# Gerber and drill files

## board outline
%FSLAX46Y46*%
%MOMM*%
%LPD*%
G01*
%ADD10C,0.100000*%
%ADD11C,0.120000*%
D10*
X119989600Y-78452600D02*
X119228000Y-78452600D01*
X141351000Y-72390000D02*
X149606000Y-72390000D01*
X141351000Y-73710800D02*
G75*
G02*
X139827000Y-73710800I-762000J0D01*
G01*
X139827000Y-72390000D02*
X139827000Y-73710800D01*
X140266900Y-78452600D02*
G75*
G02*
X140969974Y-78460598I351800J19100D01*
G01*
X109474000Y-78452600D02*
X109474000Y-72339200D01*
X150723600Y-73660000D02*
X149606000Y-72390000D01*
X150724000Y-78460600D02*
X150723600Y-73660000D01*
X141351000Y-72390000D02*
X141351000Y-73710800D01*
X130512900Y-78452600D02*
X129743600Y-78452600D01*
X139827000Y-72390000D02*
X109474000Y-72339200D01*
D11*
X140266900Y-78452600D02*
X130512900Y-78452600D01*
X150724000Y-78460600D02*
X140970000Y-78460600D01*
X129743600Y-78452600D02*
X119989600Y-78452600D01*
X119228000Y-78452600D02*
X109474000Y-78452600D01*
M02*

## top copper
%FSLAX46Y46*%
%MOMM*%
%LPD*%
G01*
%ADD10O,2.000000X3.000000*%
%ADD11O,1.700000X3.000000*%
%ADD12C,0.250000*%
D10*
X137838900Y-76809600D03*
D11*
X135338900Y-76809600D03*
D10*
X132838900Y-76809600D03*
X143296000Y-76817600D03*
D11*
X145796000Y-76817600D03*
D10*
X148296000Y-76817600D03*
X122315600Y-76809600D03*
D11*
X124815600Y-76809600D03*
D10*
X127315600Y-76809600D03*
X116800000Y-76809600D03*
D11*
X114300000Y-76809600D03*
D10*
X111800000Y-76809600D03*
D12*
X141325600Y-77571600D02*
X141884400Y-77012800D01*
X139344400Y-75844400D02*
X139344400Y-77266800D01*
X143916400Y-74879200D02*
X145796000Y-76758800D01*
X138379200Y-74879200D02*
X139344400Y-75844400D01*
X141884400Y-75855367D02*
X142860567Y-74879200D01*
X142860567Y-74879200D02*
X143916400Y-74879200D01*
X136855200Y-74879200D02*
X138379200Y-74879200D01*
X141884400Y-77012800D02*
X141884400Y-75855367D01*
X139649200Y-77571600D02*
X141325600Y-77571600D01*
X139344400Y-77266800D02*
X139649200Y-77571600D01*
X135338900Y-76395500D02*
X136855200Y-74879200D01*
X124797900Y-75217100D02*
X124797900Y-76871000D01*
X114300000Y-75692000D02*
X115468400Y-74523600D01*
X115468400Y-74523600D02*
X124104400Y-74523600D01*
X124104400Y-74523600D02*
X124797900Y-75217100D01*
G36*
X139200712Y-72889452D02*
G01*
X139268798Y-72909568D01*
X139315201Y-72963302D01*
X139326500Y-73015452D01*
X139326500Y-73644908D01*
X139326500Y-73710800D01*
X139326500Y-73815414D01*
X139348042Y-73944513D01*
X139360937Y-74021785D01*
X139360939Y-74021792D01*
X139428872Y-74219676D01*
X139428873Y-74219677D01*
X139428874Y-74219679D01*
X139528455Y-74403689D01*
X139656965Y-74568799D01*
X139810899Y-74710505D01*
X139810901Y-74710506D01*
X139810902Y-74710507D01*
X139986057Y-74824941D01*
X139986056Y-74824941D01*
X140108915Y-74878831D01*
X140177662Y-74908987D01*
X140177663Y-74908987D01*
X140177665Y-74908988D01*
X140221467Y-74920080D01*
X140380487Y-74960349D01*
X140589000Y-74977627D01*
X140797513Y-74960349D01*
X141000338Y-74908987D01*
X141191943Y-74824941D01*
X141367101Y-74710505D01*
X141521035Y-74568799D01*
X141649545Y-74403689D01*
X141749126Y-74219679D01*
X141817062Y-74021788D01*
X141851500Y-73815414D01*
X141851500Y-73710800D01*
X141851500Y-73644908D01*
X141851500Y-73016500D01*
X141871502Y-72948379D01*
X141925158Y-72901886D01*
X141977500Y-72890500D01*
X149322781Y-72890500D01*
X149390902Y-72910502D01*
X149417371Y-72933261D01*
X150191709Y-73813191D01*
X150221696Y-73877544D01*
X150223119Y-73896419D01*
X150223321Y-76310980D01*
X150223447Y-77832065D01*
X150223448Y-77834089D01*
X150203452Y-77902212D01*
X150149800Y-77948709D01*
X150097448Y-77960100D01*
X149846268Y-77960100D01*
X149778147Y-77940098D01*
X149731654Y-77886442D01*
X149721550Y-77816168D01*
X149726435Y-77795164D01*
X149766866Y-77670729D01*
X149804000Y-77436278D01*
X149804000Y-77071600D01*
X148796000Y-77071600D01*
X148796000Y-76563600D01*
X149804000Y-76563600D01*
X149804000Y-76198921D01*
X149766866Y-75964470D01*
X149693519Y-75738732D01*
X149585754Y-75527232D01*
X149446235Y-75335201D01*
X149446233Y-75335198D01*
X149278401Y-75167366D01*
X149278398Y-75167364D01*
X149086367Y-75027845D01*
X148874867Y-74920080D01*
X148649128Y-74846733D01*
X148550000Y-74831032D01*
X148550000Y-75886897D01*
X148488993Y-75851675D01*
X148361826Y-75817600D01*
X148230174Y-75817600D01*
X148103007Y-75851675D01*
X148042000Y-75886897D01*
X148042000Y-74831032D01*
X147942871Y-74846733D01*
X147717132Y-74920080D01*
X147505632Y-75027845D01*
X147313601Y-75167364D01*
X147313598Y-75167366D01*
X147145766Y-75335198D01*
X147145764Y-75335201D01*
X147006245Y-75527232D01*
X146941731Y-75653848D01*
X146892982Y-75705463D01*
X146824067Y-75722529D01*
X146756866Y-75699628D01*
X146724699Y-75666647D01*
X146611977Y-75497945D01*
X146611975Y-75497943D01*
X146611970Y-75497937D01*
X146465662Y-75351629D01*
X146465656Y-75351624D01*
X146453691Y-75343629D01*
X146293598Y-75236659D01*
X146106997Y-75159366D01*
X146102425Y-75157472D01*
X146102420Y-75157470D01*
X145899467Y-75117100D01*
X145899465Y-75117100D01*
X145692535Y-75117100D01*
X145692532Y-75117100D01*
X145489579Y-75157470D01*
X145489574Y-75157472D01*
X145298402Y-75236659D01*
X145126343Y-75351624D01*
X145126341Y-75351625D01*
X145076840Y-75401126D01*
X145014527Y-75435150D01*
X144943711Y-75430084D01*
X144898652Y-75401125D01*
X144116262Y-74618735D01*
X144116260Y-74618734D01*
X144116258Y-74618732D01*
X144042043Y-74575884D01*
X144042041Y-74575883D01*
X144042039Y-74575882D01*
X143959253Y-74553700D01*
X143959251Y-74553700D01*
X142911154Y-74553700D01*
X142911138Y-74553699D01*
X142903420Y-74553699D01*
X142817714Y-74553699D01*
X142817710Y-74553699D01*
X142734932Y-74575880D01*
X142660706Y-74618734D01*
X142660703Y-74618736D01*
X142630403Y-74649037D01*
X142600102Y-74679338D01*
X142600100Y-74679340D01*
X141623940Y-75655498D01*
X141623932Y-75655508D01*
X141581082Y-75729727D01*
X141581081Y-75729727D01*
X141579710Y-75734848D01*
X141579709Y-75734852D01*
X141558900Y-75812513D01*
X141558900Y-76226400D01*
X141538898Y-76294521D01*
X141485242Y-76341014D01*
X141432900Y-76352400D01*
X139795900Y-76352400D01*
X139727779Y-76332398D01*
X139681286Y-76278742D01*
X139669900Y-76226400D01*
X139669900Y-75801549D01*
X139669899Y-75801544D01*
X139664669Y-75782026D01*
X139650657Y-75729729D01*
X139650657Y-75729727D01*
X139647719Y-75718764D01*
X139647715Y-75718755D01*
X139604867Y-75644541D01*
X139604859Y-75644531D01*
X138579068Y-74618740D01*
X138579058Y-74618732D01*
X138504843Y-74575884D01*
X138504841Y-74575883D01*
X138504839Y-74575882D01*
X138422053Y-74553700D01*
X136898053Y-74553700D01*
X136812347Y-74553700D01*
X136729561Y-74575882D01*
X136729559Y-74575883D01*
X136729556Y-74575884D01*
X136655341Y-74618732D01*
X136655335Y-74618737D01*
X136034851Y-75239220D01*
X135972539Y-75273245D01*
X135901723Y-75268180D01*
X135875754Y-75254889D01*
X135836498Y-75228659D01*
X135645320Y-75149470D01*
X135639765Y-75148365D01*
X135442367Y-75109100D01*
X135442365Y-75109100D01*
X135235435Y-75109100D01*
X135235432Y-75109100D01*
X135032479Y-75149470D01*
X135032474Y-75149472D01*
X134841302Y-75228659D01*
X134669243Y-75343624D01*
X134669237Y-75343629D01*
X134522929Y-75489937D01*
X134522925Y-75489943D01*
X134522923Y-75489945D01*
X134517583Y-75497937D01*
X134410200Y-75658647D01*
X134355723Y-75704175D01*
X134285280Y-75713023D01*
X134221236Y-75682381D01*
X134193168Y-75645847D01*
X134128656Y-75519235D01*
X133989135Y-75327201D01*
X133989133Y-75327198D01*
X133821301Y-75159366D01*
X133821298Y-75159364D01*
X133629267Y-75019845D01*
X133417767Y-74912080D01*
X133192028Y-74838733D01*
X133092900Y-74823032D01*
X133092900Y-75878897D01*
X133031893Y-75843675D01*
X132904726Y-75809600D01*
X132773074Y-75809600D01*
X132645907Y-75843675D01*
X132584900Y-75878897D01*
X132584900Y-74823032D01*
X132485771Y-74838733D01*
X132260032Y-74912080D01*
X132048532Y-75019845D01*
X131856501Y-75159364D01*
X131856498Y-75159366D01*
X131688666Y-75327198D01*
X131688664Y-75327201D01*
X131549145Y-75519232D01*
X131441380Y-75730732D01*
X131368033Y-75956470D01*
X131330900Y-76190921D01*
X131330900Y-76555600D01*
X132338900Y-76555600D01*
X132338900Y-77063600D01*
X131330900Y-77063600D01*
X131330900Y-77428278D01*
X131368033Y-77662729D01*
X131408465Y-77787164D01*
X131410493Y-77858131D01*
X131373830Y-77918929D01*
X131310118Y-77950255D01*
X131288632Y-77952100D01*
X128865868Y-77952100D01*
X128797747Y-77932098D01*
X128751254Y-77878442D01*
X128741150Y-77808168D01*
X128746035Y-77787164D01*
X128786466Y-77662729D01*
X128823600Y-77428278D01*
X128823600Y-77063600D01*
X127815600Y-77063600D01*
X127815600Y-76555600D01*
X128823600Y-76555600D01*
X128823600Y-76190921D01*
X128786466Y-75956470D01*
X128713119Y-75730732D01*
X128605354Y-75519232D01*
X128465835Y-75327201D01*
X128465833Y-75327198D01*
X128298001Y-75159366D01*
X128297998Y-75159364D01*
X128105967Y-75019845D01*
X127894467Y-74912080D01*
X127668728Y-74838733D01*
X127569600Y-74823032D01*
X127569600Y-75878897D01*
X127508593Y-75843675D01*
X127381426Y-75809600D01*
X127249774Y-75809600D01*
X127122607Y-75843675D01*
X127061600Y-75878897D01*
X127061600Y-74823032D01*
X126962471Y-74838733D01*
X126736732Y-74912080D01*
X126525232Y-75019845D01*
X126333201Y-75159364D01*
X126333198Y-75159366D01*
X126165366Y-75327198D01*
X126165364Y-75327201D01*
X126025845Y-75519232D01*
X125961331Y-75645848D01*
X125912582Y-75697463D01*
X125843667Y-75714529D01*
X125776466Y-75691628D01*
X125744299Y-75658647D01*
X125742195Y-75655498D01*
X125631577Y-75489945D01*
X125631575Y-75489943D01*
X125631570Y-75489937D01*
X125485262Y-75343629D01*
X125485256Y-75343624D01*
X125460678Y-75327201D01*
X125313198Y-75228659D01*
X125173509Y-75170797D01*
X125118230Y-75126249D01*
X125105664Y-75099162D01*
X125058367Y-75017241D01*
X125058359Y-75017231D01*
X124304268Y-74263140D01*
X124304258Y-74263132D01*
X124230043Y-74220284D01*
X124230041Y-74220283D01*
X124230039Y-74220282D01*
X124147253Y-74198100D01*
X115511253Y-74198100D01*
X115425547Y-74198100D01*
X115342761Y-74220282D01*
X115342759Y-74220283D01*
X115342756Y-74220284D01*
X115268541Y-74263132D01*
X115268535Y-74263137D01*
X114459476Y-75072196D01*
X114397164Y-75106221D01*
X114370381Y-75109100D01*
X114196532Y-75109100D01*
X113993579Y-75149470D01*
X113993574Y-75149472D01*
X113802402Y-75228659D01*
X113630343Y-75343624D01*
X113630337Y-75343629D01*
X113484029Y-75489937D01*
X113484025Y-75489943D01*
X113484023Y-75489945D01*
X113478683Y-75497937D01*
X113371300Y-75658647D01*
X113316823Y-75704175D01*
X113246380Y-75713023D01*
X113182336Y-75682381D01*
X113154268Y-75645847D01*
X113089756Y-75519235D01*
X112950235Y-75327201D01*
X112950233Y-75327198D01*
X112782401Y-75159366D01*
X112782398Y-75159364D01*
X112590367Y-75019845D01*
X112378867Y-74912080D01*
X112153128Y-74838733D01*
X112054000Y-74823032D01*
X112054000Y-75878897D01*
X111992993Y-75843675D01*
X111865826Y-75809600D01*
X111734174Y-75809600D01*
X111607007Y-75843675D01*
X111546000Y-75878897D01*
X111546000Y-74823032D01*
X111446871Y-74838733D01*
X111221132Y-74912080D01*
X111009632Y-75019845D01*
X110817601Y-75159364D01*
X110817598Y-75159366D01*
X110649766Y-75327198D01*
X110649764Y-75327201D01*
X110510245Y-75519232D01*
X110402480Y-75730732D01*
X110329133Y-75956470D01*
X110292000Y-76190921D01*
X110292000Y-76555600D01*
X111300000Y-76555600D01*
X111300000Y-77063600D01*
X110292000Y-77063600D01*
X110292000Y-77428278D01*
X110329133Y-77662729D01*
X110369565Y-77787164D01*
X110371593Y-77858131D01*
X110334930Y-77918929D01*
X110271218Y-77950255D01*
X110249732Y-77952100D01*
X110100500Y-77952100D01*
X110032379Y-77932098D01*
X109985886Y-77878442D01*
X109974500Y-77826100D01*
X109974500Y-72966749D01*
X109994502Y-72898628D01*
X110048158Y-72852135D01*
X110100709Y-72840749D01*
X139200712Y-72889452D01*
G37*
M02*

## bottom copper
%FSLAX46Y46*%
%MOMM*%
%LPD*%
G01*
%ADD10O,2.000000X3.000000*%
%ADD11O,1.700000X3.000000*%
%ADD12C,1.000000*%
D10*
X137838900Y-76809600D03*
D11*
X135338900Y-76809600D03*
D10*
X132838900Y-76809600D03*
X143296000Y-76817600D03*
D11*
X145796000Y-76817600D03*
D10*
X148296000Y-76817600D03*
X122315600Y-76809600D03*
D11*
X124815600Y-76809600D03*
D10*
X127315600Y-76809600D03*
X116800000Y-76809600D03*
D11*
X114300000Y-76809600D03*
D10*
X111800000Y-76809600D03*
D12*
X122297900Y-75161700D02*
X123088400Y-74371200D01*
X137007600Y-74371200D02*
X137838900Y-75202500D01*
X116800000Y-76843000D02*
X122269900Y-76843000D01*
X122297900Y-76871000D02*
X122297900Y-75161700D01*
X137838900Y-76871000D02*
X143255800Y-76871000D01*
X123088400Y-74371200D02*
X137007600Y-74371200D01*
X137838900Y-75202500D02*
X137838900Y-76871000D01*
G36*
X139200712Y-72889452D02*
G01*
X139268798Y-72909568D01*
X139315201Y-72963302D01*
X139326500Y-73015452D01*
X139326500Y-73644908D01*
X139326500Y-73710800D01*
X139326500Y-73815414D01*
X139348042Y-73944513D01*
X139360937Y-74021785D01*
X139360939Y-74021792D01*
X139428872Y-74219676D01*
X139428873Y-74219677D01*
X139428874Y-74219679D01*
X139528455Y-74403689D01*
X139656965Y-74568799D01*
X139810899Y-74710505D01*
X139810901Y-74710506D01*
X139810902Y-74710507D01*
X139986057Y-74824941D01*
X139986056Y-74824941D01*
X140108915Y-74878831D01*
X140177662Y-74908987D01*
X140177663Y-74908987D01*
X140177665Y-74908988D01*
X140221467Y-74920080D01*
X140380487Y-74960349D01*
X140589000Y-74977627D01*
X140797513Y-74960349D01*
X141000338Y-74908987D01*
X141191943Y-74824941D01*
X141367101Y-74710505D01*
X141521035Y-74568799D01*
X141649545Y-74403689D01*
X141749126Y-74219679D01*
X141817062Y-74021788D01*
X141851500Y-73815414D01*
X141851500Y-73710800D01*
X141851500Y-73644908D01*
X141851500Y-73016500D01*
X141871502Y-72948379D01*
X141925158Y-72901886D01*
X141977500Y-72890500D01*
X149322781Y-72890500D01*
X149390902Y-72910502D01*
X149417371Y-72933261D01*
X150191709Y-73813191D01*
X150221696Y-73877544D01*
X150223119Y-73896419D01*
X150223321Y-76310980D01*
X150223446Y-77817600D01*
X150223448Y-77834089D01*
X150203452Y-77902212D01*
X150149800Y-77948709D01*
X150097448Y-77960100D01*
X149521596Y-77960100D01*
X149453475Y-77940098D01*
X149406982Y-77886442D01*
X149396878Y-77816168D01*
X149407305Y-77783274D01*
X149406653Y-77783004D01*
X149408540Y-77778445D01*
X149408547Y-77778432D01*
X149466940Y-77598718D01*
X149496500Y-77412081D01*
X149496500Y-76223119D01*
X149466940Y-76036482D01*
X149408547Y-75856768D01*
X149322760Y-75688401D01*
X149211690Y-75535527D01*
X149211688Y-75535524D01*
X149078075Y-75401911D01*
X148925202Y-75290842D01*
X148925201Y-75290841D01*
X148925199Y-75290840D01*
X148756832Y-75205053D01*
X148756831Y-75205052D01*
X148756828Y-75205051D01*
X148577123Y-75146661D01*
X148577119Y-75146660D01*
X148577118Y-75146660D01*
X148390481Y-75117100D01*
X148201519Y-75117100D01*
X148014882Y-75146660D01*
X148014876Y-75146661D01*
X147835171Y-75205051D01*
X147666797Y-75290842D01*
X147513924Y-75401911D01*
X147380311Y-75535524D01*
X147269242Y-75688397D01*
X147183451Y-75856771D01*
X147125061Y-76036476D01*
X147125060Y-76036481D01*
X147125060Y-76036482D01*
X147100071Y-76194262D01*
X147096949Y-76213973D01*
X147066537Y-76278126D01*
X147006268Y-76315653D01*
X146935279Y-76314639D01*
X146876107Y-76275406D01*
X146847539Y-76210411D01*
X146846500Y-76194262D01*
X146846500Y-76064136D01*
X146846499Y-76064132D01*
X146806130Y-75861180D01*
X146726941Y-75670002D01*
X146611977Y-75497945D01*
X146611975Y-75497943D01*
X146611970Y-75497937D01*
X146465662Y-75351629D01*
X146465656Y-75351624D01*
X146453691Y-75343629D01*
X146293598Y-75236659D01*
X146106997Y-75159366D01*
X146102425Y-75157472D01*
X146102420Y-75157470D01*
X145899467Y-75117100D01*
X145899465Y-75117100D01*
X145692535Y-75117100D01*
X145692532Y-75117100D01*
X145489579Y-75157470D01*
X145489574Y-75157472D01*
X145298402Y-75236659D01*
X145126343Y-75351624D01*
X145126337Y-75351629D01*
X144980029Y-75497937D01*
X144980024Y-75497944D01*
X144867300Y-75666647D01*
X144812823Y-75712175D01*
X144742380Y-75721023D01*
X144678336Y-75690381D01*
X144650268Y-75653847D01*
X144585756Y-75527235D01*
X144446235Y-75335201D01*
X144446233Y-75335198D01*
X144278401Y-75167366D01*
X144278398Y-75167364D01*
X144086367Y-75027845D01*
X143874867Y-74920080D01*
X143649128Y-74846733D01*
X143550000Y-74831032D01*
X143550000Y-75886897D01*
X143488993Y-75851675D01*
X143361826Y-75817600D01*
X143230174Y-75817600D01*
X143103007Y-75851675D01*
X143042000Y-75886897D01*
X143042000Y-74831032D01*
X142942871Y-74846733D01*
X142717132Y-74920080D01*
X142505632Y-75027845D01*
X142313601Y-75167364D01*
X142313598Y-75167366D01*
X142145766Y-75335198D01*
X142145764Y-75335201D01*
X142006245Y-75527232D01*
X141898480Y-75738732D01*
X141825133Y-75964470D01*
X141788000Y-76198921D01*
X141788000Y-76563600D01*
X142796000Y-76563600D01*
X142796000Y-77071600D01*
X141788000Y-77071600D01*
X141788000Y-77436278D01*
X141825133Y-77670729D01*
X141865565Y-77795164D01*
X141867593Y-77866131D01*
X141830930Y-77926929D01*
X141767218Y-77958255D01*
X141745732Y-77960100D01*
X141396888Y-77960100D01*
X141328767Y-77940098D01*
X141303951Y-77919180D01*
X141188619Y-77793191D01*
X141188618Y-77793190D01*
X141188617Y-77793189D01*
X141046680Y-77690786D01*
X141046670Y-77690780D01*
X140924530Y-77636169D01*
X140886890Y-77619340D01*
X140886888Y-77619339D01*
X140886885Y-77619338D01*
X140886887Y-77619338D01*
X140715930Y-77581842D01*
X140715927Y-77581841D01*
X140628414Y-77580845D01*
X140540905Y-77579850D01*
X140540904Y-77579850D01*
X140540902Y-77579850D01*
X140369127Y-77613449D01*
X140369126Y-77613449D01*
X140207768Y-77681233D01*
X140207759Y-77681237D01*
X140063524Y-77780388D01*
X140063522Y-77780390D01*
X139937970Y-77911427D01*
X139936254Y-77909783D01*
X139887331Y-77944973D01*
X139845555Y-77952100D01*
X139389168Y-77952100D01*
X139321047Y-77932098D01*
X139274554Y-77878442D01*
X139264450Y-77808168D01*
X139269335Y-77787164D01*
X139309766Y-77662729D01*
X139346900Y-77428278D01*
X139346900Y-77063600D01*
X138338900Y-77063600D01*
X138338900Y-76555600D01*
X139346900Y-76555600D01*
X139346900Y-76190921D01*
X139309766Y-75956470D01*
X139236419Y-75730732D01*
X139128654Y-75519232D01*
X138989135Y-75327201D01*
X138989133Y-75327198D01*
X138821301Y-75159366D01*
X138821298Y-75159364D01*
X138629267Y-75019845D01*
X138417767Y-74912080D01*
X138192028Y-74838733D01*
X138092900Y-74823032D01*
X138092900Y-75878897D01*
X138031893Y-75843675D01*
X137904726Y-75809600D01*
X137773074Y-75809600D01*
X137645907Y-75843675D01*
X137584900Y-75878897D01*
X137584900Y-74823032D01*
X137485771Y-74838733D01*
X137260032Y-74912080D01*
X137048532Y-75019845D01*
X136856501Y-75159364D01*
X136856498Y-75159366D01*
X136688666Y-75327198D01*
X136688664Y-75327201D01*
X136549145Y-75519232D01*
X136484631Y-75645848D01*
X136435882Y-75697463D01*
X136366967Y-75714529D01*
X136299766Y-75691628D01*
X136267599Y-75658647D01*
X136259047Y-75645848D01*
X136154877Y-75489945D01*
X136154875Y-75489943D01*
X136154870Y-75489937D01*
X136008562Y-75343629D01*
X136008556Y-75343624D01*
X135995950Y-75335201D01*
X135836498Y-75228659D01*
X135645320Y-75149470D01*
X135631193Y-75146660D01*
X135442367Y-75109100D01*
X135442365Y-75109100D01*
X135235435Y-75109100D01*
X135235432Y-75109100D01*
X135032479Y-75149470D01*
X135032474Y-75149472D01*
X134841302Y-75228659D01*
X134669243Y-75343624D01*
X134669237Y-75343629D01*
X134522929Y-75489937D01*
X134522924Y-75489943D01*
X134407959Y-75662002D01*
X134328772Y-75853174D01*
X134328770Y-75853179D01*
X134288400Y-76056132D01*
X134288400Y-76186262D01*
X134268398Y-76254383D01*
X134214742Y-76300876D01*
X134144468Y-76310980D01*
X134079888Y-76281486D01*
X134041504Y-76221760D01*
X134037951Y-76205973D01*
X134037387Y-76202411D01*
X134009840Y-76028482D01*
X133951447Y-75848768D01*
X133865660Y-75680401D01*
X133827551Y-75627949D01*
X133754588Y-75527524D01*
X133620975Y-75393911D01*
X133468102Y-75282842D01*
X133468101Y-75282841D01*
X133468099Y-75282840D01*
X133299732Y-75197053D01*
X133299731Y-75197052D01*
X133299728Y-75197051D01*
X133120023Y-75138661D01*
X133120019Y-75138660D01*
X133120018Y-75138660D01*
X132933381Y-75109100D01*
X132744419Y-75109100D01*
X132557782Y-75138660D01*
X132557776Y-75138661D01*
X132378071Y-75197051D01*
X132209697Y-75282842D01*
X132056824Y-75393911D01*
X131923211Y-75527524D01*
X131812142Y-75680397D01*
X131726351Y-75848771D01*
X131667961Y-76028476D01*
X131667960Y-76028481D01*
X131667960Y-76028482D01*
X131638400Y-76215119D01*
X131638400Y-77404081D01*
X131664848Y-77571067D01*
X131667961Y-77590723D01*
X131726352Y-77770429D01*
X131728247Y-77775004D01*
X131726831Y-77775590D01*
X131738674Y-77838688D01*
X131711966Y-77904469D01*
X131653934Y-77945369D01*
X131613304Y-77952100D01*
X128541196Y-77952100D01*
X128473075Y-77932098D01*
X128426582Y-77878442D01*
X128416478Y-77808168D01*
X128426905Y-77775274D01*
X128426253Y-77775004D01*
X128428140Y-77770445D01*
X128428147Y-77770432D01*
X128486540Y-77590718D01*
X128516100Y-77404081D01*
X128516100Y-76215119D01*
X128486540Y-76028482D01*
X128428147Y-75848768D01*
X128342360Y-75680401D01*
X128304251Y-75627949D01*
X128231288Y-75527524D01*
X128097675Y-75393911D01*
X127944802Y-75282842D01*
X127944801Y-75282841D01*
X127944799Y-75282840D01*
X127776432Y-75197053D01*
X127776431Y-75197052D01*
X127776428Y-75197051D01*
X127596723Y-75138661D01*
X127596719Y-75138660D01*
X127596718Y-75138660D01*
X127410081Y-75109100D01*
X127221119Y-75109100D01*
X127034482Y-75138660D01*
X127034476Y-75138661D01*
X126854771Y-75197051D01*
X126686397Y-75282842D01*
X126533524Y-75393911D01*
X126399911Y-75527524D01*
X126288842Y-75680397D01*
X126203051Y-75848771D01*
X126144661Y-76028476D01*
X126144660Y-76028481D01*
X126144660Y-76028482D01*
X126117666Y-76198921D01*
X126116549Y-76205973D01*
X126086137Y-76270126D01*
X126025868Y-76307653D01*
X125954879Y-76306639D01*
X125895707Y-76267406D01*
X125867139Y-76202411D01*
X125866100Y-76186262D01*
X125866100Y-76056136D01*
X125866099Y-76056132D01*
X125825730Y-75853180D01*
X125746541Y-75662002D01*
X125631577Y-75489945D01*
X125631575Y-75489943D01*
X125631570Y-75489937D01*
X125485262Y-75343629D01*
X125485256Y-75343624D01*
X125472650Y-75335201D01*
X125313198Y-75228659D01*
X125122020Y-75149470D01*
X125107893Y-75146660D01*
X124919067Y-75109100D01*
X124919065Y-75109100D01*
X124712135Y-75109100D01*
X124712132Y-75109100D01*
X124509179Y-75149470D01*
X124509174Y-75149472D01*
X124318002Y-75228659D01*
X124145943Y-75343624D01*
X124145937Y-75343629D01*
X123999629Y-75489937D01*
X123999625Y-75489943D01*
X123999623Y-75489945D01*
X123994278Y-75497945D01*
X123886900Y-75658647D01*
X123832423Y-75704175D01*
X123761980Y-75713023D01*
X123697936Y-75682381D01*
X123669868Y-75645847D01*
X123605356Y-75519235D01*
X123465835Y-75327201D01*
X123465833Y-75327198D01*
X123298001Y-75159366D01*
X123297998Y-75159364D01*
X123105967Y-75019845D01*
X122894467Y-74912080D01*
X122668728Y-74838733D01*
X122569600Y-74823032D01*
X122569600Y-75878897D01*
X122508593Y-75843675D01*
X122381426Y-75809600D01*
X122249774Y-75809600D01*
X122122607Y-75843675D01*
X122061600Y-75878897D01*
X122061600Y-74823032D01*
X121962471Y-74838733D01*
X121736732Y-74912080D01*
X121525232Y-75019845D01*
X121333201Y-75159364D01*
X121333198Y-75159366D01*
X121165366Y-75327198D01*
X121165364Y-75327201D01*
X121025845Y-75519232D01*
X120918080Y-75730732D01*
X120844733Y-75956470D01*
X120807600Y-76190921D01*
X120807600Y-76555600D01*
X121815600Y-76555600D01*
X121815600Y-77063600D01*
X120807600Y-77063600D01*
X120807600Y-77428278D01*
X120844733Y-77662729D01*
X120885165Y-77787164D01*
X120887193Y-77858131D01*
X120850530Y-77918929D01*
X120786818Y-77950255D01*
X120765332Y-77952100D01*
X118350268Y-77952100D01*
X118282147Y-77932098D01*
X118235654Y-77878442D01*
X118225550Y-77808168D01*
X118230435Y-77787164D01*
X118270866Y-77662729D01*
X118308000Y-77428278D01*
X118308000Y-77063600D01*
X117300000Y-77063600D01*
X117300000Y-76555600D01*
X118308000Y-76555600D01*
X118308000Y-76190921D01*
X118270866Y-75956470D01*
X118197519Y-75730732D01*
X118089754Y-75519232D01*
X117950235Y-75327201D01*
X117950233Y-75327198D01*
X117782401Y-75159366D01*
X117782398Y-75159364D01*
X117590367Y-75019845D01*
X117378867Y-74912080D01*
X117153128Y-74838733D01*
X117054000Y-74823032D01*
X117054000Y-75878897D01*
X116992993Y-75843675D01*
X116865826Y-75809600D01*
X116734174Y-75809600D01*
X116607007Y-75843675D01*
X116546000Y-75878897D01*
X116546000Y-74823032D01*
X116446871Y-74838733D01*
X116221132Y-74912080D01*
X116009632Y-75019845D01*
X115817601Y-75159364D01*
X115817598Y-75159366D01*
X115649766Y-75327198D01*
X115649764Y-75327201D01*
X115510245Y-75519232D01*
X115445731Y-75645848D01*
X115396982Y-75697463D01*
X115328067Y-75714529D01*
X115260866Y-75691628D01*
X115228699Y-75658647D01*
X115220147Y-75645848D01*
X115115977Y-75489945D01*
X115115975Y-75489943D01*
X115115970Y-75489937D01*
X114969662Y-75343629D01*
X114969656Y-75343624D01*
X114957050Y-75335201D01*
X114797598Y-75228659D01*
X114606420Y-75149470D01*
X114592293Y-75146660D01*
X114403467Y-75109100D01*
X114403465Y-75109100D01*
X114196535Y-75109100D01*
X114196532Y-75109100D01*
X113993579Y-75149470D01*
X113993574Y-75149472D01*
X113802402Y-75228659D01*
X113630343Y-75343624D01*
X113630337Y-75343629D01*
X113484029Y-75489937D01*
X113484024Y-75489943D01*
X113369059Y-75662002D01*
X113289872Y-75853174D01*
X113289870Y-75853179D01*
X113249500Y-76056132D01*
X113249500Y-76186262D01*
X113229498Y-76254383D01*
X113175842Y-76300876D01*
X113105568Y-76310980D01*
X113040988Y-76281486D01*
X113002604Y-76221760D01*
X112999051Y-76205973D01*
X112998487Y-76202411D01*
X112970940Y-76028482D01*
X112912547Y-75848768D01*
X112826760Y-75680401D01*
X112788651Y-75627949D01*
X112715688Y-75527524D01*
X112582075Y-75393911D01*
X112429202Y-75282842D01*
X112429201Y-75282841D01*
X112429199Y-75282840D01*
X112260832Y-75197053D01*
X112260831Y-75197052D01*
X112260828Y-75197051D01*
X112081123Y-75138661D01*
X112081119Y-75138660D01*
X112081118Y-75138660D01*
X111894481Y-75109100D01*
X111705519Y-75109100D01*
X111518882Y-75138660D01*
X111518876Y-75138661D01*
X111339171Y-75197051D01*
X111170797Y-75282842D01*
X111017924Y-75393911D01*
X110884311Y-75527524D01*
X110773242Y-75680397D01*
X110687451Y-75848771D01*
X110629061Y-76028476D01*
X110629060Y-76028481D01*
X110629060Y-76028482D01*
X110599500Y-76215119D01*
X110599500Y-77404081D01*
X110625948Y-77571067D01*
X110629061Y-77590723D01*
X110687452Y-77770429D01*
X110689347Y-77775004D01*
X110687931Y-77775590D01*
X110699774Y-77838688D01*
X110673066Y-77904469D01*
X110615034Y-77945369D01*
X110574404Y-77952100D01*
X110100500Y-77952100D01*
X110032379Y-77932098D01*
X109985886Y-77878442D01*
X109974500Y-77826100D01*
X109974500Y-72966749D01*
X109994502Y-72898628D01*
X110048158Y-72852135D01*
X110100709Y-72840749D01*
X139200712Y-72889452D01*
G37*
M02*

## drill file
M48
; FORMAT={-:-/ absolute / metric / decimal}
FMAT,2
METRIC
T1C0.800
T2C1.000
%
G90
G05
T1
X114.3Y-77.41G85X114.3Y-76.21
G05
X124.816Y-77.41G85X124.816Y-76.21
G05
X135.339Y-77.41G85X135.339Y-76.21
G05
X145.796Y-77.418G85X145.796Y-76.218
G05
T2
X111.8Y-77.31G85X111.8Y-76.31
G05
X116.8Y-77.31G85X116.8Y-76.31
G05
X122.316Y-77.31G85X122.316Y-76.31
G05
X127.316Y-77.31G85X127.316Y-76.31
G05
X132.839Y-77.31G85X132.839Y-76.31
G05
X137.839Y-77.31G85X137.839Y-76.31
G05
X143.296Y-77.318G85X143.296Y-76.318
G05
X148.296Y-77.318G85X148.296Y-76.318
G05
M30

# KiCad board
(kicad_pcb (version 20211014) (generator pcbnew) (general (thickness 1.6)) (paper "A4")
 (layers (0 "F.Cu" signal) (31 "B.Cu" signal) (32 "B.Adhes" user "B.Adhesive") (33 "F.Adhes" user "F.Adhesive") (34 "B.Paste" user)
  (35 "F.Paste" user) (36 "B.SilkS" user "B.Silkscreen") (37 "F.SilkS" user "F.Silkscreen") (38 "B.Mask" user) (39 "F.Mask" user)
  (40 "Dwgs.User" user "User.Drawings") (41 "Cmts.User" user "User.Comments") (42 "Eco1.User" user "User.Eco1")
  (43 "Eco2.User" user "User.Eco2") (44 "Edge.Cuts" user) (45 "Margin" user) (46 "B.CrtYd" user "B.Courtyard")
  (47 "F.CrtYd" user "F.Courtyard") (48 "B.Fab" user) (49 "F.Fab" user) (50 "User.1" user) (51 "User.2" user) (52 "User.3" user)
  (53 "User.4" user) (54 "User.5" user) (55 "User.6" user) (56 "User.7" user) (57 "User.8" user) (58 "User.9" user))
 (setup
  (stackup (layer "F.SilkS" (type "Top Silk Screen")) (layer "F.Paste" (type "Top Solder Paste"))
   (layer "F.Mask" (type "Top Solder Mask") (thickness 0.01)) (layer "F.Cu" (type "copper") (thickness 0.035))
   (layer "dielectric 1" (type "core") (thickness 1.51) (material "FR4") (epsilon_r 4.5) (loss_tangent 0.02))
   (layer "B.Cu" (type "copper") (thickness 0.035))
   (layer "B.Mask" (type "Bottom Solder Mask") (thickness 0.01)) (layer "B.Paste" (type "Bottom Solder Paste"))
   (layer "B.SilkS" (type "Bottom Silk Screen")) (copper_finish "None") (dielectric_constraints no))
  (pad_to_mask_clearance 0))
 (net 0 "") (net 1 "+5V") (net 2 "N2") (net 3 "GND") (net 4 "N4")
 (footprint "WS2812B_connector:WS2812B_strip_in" (layer "F.Cu") (at 135.3389 77.3096 180)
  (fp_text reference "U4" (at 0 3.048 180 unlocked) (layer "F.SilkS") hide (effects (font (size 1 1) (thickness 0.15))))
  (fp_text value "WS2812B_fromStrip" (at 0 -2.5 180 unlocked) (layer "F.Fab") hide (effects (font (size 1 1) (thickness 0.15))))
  (fp_line (start -4.928 -1.143) (end 4.826 -1.143) (layer "Edge.Cuts") (width 0.12))
  (pad "1" thru_hole oval (at -2.5 0.5 180) (size 2 3) (drill oval 1 2) (layers *.Cu *.Mask) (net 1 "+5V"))
  (pad "2" thru_hole oval (at 0 0.5 180) (size 1.7 3) (drill oval 0.8 2) (layers *.Cu *.Mask) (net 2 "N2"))
  (pad "3" thru_hole oval (at 2.5 0.5 180) (size 2 3) (drill oval 1 2) (layers *.Cu *.Mask) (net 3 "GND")))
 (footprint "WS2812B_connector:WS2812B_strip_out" (layer "F.Cu") (at 145.796 77.3176 180)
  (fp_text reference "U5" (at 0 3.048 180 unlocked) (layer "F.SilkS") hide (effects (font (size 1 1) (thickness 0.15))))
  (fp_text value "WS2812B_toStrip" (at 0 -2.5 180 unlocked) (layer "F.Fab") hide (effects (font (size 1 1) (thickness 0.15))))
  (fp_line (start -4.928 -1.143) (end 4.826 -1.143) (layer "Edge.Cuts") (width 0.12))
  (pad "1" thru_hole oval (at 2.5 0.5 180) (size 2 3) (drill oval 1 2) (layers *.Cu *.Mask) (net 1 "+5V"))
  (pad "2" thru_hole oval (at 0 0.5 180) (size 1.7 3) (drill oval 0.8 2) (layers *.Cu *.Mask) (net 2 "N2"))
  (pad "3" thru_hole oval (at -2.5 0.5 180) (size 2 3) (drill oval 1 2) (layers *.Cu *.Mask) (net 3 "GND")))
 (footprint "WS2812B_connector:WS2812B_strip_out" (layer "F.Cu") (at 124.8156 77.3096 180)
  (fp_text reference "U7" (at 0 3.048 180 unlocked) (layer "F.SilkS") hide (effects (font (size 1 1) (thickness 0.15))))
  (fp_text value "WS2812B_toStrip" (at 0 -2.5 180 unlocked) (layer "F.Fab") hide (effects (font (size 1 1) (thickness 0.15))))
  (fp_line (start -4.928 -1.143) (end 4.826 -1.143) (layer "Edge.Cuts") (width 0.12))
  (pad "1" thru_hole oval (at 2.5 0.5 180) (size 2 3) (drill oval 1 2) (layers *.Cu *.Mask) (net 1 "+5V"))
  (pad "2" thru_hole oval (at 0 0.5 180) (size 1.7 3) (drill oval 0.8 2) (layers *.Cu *.Mask) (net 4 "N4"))
  (pad "3" thru_hole oval (at -2.5 0.5 180) (size 2 3) (drill oval 1 2) (layers *.Cu *.Mask) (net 3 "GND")))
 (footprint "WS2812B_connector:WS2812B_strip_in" (layer "F.Cu") (at 114.3 77.3096 180)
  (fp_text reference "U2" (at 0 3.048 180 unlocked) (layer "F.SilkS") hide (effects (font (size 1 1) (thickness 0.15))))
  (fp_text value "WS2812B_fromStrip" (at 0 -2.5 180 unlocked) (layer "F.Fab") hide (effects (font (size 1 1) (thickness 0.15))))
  (fp_line (start -4.928 -1.143) (end 4.826 -1.143) (layer "Edge.Cuts") (width 0.12))
  (pad "1" thru_hole oval (at -2.5 0.5 180) (size 2 3) (drill oval 1 2) (layers *.Cu *.Mask) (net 1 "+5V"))
  (pad "2" thru_hole oval (at 0 0.5 180) (size 1.7 3) (drill oval 0.8 2) (layers *.Cu *.Mask) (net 4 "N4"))
  (pad "3" thru_hole oval (at 2.5 0.5 180) (size 2 3) (drill oval 1 2) (layers *.Cu *.Mask) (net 3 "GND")))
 (gr_line (start 119.9896 78.4526) (end 119.228 78.4526) (layer "Edge.Cuts") (width 0.1))
 (gr_line (start 141.351 72.39) (end 149.606 72.39) (layer "Edge.Cuts") (width 0.1))
 (gr_arc (start 141.351 73.7108) (mid 140.589 74.4728) (end 139.827 73.7108) (layer "Edge.Cuts") (width 0.1))
 (gr_line (start 139.827 72.39) (end 139.827 73.7108) (layer "Edge.Cuts") (width 0.1))
 (gr_arc (start 140.2669 78.4526) (mid 140.622721 78.081232) (end 140.97 78.4606) (layer "Edge.Cuts") (width 0.1))
 (gr_line (start 109.474 78.4526) (end 109.474 72.3392) (layer "Edge.Cuts") (width 0.1))
 (gr_line (start 150.7236 73.66) (end 149.606 72.39) (layer "Edge.Cuts") (width 0.1))
 (gr_line (start 150.724 78.4606) (end 150.7236 73.66) (layer "Edge.Cuts") (width 0.1))
 (gr_line (start 141.351 72.39) (end 141.351 73.7108) (layer "Edge.Cuts") (width 0.1))
 (gr_line (start 130.5129 78.4526) (end 129.7436 78.4526) (layer "Edge.Cuts") (width 0.1))
 (gr_line (start 139.827 72.39) (end 109.474 72.3392) (layer "Edge.Cuts") (width 0.1))
 (segment (start 122.2979 75.1617) (end 123.0884 74.3712) (width 1) (layer "B.Cu") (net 1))
 (segment (start 137.0076 74.3712) (end 137.8389 75.2025) (width 1) (layer "B.Cu") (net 1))
 (segment (start 116.8 76.843) (end 122.2699 76.843) (width 1) (layer "B.Cu") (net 1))
 (segment (start 122.2979 76.871) (end 122.2979 75.1617) (width 1) (layer "B.Cu") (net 1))
 (segment (start 137.8389 76.871) (end 143.2558 76.871) (width 1) (layer "B.Cu") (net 1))
 (segment (start 123.0884 74.3712) (end 137.0076 74.3712) (width 1) (layer "B.Cu") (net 1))
 (segment (start 137.8389 75.2025) (end 137.8389 76.871) (width 1) (layer "B.Cu") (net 1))
 (segment (start 141.3256 77.5716) (end 141.8844 77.0128) (width 0.25) (layer "F.Cu") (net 2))
 (segment (start 139.3444 75.8444) (end 139.3444 77.2668) (width 0.25) (layer "F.Cu") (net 2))
 (segment (start 143.9164 74.8792) (end 145.796 76.7588) (width 0.25) (layer "F.Cu") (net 2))
 (segment (start 138.3792 74.8792) (end 139.3444 75.8444) (width 0.25) (layer "F.Cu") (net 2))
 (segment (start 141.8844 75.855367) (end 142.860567 74.8792) (width 0.25) (layer "F.Cu") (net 2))
 (segment (start 142.860567 74.8792) (end 143.9164 74.8792) (width 0.25) (layer "F.Cu") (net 2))
 (segment (start 136.8552 74.8792) (end 138.3792 74.8792) (width 0.25) (layer "F.Cu") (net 2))
 (segment (start 141.8844 77.0128) (end 141.8844 75.855367) (width 0.25) (layer "F.Cu") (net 2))
 (segment (start 139.6492 77.5716) (end 141.3256 77.5716) (width 0.25) (layer "F.Cu") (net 2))
 (segment (start 139.3444 77.2668) (end 139.6492 77.5716) (width 0.25) (layer "F.Cu") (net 2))
 (segment (start 135.3389 76.3955) (end 136.8552 74.8792) (width 0.25) (layer "F.Cu") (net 2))
 (segment (start 124.7979 75.2171) (end 124.7979 76.871) (width 0.25) (layer "F.Cu") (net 4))
 (segment (start 114.3 75.692) (end 115.4684 74.5236) (width 0.25) (layer "F.Cu") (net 4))
 (segment (start 115.4684 74.5236) (end 124.1044 74.5236) (width 0.25) (layer "F.Cu") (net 4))
 (segment (start 124.1044 74.5236) (end 124.7979 75.2171) (width 0.25) (layer "F.Cu") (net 4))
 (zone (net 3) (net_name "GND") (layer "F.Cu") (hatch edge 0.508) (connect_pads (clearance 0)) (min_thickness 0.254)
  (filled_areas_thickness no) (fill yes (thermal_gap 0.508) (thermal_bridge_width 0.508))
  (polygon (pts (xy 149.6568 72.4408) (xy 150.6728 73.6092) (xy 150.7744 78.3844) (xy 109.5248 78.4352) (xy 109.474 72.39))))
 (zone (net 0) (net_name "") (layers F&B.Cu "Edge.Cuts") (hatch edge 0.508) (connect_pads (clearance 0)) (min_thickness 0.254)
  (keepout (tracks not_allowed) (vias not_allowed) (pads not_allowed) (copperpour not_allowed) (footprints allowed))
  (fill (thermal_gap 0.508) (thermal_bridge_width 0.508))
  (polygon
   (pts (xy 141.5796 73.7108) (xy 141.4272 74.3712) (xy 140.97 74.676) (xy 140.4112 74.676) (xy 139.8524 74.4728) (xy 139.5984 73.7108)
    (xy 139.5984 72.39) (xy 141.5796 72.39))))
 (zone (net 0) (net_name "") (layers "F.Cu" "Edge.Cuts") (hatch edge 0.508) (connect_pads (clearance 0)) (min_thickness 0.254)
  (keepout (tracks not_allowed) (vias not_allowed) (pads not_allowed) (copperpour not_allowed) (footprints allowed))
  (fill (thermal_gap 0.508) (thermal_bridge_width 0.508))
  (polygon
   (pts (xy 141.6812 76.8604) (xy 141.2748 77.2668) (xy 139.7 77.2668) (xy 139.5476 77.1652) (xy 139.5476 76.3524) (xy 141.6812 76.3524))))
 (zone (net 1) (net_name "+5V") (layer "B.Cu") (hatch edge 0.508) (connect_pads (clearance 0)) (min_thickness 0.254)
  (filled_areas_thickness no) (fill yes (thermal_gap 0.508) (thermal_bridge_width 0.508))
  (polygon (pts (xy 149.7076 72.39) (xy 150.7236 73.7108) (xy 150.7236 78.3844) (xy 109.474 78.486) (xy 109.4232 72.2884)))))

